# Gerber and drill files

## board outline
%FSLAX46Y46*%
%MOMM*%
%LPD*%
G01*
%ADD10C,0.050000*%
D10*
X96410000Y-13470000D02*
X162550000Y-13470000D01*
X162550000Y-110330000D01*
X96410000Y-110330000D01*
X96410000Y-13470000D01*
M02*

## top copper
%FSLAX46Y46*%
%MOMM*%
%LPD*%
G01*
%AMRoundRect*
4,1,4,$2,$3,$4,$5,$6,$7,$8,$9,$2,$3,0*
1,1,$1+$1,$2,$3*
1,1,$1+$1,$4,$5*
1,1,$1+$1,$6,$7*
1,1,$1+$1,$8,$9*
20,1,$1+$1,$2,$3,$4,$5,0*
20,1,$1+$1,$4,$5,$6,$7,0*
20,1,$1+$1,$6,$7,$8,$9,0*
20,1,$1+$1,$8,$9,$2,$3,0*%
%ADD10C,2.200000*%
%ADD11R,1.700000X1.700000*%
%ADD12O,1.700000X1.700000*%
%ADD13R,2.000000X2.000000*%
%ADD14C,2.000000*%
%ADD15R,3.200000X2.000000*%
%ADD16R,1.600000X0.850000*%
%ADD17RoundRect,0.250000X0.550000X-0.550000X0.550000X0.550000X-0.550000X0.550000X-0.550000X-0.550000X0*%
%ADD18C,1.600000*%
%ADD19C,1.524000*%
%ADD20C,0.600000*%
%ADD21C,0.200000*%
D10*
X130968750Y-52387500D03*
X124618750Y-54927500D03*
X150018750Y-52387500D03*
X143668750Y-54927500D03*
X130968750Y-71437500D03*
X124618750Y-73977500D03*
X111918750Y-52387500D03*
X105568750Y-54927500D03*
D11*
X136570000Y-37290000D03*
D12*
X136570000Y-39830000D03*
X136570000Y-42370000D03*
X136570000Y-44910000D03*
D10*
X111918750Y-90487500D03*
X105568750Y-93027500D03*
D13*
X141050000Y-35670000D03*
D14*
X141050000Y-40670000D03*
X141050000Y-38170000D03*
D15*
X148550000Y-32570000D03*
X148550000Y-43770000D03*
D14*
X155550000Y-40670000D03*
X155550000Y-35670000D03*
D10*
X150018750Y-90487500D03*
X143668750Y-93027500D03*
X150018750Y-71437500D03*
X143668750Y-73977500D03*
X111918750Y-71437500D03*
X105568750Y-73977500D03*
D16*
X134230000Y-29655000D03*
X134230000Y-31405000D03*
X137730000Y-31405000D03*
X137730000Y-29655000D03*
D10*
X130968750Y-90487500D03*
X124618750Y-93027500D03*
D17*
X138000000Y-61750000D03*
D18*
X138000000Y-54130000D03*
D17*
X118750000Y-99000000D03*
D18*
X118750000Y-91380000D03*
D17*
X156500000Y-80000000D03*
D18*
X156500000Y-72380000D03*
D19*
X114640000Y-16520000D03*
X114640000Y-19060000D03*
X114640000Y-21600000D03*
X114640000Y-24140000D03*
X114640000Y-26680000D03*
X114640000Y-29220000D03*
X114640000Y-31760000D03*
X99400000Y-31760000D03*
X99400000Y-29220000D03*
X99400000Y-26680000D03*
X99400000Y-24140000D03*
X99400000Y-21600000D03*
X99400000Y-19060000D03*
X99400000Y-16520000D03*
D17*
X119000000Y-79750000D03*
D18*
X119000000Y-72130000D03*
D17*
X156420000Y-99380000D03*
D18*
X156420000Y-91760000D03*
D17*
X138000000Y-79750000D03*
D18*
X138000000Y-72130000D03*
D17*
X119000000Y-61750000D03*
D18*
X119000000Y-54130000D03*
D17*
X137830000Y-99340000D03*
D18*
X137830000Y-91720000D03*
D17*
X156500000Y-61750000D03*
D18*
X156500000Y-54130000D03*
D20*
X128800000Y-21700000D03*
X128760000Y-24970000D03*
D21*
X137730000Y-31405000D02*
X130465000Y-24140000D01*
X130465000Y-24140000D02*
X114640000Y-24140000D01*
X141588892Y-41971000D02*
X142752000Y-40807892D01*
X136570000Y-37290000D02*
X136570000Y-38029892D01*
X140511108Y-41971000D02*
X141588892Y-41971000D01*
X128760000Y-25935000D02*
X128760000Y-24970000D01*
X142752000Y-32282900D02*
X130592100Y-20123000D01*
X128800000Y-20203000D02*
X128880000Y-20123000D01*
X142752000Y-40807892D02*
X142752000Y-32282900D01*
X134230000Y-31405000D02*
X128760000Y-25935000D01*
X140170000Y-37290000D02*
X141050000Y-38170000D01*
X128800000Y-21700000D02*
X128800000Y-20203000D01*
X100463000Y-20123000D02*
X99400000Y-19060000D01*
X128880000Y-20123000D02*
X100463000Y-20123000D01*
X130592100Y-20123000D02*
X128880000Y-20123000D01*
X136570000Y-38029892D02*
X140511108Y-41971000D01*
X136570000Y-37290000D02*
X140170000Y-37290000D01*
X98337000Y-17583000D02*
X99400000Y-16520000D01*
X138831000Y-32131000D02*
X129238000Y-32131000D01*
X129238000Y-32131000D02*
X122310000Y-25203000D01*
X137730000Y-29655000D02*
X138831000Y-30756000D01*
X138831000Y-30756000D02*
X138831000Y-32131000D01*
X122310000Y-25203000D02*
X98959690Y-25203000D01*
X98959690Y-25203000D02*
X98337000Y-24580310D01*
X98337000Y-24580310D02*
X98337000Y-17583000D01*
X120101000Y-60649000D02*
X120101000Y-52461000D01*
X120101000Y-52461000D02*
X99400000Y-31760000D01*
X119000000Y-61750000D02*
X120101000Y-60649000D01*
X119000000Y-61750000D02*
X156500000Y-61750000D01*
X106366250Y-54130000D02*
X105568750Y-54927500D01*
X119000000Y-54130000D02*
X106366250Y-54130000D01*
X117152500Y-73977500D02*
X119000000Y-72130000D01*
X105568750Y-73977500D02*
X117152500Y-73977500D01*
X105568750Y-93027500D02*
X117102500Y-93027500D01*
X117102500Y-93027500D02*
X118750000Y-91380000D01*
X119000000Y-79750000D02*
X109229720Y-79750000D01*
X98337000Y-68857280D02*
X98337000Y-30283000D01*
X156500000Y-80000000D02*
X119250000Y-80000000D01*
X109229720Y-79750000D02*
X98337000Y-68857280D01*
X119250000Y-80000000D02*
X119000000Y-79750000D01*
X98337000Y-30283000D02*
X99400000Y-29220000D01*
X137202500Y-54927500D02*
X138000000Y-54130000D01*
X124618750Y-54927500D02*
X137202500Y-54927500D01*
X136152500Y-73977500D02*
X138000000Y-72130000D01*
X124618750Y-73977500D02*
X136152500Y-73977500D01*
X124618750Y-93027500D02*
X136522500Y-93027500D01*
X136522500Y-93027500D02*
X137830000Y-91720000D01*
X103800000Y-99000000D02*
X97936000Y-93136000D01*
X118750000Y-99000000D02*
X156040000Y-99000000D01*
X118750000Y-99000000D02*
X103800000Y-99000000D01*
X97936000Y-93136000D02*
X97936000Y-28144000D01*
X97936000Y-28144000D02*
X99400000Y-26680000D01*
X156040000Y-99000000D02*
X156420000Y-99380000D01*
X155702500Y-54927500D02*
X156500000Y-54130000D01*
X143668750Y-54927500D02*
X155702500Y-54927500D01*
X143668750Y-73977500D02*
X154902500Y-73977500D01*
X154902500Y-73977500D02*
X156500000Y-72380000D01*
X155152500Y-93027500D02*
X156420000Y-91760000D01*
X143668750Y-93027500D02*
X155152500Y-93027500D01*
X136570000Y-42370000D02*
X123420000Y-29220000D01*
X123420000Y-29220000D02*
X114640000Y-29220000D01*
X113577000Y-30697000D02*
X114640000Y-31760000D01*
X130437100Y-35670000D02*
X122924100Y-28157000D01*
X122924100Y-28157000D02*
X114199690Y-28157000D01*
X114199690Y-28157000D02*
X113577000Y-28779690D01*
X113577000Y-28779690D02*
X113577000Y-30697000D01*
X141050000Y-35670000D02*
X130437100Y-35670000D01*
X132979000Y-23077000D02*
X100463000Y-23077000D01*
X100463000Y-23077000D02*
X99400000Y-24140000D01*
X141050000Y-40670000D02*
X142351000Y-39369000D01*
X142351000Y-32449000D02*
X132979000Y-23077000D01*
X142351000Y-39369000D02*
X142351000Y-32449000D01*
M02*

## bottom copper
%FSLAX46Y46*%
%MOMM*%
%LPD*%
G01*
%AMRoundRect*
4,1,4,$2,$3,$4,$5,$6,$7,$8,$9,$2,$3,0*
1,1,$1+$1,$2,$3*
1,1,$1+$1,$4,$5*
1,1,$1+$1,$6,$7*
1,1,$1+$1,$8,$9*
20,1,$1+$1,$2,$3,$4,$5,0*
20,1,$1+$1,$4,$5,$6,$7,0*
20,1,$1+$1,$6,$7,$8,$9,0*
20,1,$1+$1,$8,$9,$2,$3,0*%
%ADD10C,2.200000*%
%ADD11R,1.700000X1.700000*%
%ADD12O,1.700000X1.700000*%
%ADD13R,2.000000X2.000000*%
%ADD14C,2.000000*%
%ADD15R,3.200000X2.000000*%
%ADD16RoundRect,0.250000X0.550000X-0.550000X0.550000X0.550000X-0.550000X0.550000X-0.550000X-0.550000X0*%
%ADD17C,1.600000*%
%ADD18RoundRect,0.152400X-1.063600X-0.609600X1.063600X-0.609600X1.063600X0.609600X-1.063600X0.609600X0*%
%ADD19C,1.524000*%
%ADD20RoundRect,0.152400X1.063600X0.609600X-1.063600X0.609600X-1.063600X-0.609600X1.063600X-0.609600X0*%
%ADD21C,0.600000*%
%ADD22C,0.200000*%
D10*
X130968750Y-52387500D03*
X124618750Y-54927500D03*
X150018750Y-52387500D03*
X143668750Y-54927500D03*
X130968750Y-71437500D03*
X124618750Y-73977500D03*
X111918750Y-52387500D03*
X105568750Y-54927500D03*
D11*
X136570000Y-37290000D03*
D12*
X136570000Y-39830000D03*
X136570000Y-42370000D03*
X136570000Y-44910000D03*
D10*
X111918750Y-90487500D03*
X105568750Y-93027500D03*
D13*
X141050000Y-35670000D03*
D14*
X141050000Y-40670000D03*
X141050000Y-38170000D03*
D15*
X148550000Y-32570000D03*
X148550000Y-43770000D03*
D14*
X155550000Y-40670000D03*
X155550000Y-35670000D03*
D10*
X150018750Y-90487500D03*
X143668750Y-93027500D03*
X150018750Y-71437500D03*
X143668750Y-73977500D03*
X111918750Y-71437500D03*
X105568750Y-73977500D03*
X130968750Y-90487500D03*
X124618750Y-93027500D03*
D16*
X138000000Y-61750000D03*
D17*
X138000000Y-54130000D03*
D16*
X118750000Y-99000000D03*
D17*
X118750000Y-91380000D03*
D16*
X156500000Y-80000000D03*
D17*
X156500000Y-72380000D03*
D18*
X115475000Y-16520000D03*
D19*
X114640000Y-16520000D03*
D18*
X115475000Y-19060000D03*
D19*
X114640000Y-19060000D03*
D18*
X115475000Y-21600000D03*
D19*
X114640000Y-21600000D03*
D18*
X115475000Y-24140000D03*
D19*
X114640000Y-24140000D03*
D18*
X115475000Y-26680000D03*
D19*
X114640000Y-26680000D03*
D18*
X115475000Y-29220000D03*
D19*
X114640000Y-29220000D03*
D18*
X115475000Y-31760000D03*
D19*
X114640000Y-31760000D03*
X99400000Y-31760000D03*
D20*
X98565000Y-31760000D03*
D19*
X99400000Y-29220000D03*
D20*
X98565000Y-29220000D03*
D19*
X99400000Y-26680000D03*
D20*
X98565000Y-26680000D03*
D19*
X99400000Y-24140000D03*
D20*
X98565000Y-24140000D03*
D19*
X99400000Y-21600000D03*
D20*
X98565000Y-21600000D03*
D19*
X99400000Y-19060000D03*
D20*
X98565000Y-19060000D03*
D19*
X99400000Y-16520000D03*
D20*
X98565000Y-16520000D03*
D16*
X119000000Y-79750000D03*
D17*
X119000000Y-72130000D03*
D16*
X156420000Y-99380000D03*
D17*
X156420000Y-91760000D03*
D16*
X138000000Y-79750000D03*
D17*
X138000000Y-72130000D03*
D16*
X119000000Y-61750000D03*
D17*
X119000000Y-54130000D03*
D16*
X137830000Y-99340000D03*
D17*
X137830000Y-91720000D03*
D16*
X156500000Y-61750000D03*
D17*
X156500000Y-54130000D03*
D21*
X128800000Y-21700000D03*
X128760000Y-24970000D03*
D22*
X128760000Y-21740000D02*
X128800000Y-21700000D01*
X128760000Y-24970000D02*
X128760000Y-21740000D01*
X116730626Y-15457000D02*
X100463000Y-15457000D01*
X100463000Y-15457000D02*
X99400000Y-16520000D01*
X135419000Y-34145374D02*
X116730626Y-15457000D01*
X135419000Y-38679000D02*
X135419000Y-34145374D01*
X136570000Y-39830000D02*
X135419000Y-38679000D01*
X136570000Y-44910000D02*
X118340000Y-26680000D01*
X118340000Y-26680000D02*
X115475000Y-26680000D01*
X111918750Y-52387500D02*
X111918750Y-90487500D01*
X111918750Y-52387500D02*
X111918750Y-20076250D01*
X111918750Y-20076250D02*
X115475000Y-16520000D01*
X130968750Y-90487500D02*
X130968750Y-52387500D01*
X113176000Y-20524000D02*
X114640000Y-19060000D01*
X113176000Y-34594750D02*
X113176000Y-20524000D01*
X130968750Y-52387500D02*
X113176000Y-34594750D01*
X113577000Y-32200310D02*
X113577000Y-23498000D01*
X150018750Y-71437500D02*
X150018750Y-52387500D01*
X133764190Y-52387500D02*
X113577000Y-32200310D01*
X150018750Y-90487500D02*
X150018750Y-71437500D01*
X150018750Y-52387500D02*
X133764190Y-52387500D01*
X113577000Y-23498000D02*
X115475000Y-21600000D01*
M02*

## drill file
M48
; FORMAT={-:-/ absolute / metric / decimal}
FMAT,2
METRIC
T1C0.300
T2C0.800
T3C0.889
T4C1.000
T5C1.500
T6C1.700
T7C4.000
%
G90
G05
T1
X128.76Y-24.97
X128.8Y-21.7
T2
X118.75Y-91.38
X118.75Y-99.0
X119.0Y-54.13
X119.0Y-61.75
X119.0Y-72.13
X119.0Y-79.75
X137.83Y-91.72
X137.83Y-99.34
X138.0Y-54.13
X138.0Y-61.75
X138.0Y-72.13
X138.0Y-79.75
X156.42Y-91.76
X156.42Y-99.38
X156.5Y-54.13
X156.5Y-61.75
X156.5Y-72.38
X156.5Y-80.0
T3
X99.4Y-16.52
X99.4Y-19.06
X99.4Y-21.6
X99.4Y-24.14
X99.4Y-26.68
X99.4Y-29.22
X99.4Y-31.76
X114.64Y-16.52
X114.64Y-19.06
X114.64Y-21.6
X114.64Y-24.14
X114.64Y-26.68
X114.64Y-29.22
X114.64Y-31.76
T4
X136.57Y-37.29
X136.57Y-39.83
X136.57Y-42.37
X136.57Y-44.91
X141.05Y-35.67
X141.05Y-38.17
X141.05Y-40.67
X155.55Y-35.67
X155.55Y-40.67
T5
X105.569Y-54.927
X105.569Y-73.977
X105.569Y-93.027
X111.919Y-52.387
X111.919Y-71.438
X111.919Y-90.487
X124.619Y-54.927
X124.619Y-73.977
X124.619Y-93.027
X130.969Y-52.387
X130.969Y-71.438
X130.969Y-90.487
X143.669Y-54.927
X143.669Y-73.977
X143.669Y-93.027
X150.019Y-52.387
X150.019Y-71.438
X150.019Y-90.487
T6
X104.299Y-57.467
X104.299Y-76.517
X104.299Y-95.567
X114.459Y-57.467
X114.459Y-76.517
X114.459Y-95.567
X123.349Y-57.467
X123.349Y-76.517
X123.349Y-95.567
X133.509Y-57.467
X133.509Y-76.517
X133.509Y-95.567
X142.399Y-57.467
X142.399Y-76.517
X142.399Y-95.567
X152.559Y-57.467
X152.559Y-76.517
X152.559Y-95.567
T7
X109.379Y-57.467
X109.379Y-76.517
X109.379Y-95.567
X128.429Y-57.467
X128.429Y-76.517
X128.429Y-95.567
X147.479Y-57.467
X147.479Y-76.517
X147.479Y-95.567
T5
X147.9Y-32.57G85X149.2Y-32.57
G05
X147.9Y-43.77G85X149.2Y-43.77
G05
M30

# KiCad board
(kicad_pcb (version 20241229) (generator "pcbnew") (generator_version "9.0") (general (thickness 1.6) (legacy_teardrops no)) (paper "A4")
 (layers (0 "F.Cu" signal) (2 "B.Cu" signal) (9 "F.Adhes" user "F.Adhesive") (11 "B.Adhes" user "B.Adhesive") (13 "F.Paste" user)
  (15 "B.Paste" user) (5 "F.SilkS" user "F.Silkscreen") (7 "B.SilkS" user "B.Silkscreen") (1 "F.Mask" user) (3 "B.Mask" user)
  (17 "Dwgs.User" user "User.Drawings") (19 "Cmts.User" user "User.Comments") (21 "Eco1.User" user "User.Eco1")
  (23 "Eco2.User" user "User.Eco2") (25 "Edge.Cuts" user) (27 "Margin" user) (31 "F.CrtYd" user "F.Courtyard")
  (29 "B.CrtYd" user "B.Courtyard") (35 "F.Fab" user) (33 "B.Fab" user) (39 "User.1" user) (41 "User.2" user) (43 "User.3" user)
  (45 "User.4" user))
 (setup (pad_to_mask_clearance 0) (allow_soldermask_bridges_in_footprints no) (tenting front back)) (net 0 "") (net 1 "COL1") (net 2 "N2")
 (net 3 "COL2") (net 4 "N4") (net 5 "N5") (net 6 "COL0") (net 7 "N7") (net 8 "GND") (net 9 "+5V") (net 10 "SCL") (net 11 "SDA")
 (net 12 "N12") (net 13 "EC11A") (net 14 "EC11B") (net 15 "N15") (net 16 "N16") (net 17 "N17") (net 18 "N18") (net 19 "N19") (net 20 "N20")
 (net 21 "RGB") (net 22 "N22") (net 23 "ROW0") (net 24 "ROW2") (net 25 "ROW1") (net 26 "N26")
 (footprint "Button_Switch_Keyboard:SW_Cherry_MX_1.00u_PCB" (layer "F.Cu") (at 130.96875 52.3875)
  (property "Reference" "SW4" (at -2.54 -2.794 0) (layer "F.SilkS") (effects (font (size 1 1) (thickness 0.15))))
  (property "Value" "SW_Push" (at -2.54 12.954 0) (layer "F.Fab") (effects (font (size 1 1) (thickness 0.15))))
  (pad "" np_thru_hole circle (at -7.62 5.08) (size 1.7 1.7) (drill 1.7) (layers "*.Cu" "*.Mask"))
  (pad "" np_thru_hole circle (at -2.54 5.08) (size 4 4) (drill 4) (layers "*.Cu" "*.Mask"))
  (pad "" np_thru_hole circle (at 2.54 5.08) (size 1.7 1.7) (drill 1.7) (layers "*.Cu" "*.Mask"))
  (pad "1" thru_hole circle (at 0 0) (size 2.2 2.2) (drill 1.5) (layers "*.Cu" "*.Mask") (remove_unused_layers no) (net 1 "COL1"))
  (pad "2" thru_hole circle (at -6.35 2.54) (size 2.2 2.2) (drill 1.5) (layers "*.Cu" "*.Mask") (remove_unused_layers no) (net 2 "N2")))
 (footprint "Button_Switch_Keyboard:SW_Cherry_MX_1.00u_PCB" (layer "F.Cu") (at 150.01875 52.3875)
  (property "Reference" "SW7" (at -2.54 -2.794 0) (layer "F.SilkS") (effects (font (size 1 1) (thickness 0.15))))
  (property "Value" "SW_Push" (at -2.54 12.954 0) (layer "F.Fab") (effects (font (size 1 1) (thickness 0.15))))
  (pad "" np_thru_hole circle (at -7.62 5.08) (size 1.7 1.7) (drill 1.7) (layers "*.Cu" "*.Mask"))
  (pad "" np_thru_hole circle (at -2.54 5.08) (size 4 4) (drill 4) (layers "*.Cu" "*.Mask"))
  (pad "" np_thru_hole circle (at 2.54 5.08) (size 1.7 1.7) (drill 1.7) (layers "*.Cu" "*.Mask"))
  (pad "1" thru_hole circle (at 0 0) (size 2.2 2.2) (drill 1.5) (layers "*.Cu" "*.Mask") (remove_unused_layers no) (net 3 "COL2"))
  (pad "2" thru_hole circle (at -6.35 2.54) (size 2.2 2.2) (drill 1.5) (layers "*.Cu" "*.Mask") (remove_unused_layers no) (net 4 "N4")))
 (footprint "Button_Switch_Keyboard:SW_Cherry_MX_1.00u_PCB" (layer "F.Cu") (at 130.96875 71.4375)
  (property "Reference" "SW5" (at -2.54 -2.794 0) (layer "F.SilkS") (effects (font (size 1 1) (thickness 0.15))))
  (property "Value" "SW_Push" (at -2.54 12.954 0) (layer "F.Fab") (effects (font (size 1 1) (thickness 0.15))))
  (pad "" np_thru_hole circle (at -7.62 5.08) (size 1.7 1.7) (drill 1.7) (layers "*.Cu" "*.Mask"))
  (pad "" np_thru_hole circle (at -2.54 5.08) (size 4 4) (drill 4) (layers "*.Cu" "*.Mask"))
  (pad "" np_thru_hole circle (at 2.54 5.08) (size 1.7 1.7) (drill 1.7) (layers "*.Cu" "*.Mask"))
  (pad "1" thru_hole circle (at 0 0) (size 2.2 2.2) (drill 1.5) (layers "*.Cu" "*.Mask") (remove_unused_layers no) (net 1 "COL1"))
  (pad "2" thru_hole circle (at -6.35 2.54) (size 2.2 2.2) (drill 1.5) (layers "*.Cu" "*.Mask") (remove_unused_layers no) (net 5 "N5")))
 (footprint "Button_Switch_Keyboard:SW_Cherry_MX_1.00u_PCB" (layer "F.Cu") (at 111.91875 52.3875)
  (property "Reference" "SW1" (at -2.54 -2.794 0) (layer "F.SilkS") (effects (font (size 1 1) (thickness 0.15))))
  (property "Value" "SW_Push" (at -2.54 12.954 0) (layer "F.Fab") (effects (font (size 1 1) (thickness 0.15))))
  (pad "" np_thru_hole circle (at -7.62 5.08) (size 1.7 1.7) (drill 1.7) (layers "*.Cu" "*.Mask"))
  (pad "" np_thru_hole circle (at -2.54 5.08) (size 4 4) (drill 4) (layers "*.Cu" "*.Mask"))
  (pad "" np_thru_hole circle (at 2.54 5.08) (size 1.7 1.7) (drill 1.7) (layers "*.Cu" "*.Mask"))
  (pad "1" thru_hole circle (at 0 0) (size 2.2 2.2) (drill 1.5) (layers "*.Cu" "*.Mask") (remove_unused_layers no) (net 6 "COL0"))
  (pad "2" thru_hole circle (at -6.35 2.54) (size 2.2 2.2) (drill 1.5) (layers "*.Cu" "*.Mask") (remove_unused_layers no) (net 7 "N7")))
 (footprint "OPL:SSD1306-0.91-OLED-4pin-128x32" (layer "F.Cu") (at 100.07 35.1)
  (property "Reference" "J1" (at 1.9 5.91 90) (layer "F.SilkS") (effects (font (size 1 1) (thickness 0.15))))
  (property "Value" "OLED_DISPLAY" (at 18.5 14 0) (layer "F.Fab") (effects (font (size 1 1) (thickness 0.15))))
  (pad "1" thru_hole rect (at 36.5 2.19) (size 1.7 1.7) (drill 1) (layers "*.Cu" "*.Mask") (remove_unused_layers no) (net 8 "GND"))
  (pad "2" thru_hole oval (at 36.5 4.73) (size 1.7 1.7) (drill 1) (layers "*.Cu" "*.Mask") (remove_unused_layers no) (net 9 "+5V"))
  (pad "3" thru_hole oval (at 36.5 7.27) (size 1.7 1.7) (drill 1) (layers "*.Cu" "*.Mask") (remove_unused_layers no) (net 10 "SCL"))
  (pad "4" thru_hole oval (at 36.5 9.81) (size 1.7 1.7) (drill 1) (layers "*.Cu" "*.Mask") (remove_unused_layers no) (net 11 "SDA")))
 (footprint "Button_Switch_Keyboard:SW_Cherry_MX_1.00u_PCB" (layer "F.Cu") (at 111.91875 90.4875)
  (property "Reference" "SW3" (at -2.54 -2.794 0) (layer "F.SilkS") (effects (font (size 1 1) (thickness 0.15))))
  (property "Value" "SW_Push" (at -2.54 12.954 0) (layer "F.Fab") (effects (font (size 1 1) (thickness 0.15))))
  (pad "" np_thru_hole circle (at -7.62 5.08) (size 1.7 1.7) (drill 1.7) (layers "*.Cu" "*.Mask"))
  (pad "" np_thru_hole circle (at -2.54 5.08) (size 4 4) (drill 4) (layers "*.Cu" "*.Mask"))
  (pad "" np_thru_hole circle (at 2.54 5.08) (size 1.7 1.7) (drill 1.7) (layers "*.Cu" "*.Mask"))
  (pad "1" thru_hole circle (at 0 0) (size 2.2 2.2) (drill 1.5) (layers "*.Cu" "*.Mask") (remove_unused_layers no) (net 6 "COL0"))
  (pad "2" thru_hole circle (at -6.35 2.54) (size 2.2 2.2) (drill 1.5) (layers "*.Cu" "*.Mask") (remove_unused_layers no) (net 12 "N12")))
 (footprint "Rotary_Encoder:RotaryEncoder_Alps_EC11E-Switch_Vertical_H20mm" (layer "F.Cu") (at 141.05 35.67)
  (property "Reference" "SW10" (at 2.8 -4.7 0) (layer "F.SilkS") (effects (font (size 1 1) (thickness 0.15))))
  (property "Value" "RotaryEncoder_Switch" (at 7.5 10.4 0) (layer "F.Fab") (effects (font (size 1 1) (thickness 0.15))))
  (pad "A" thru_hole rect (at 0 0) (size 2 2) (drill 1) (layers "*.Cu" "*.Mask") (remove_unused_layers no) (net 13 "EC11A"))
  (pad "B" thru_hole circle (at 0 5) (size 2 2) (drill 1) (layers "*.Cu" "*.Mask") (remove_unused_layers no) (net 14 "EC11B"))
  (pad "C" thru_hole circle (at 0 2.5) (size 2 2) (drill 1) (layers "*.Cu" "*.Mask") (remove_unused_layers no) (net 8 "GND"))
  (pad "MP" thru_hole rect (at 7.5 -3.1) (size 3.2 2) (drill oval 2.8 1.5) (layers "*.Cu" "*.Mask") (remove_unused_layers no))
  (pad "MP" thru_hole rect (at 7.5 8.1) (size 3.2 2) (drill oval 2.8 1.5) (layers "*.Cu" "*.Mask") (remove_unused_layers no))
  (pad "S1" thru_hole circle (at 14.5 5) (size 2 2) (drill 1) (layers "*.Cu" "*.Mask") (remove_unused_layers no) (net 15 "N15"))
  (pad "S2" thru_hole circle (at 14.5 0) (size 2 2) (drill 1) (layers "*.Cu" "*.Mask") (remove_unused_layers no) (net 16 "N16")))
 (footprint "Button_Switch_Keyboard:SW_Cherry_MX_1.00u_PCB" (layer "F.Cu") (at 150.01875 90.4875)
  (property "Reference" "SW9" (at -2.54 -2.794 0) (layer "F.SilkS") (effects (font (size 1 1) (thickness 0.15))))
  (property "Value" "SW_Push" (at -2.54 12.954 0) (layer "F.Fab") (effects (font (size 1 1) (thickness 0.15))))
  (pad "" np_thru_hole circle (at -7.62 5.08) (size 1.7 1.7) (drill 1.7) (layers "*.Cu" "*.Mask"))
  (pad "" np_thru_hole circle (at -2.54 5.08) (size 4 4) (drill 4) (layers "*.Cu" "*.Mask"))
  (pad "" np_thru_hole circle (at 2.54 5.08) (size 1.7 1.7) (drill 1.7) (layers "*.Cu" "*.Mask"))
  (pad "1" thru_hole circle (at 0 0) (size 2.2 2.2) (drill 1.5) (layers "*.Cu" "*.Mask") (remove_unused_layers no) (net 3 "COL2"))
  (pad "2" thru_hole circle (at -6.35 2.54) (size 2.2 2.2) (drill 1.5) (layers "*.Cu" "*.Mask") (remove_unused_layers no) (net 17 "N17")))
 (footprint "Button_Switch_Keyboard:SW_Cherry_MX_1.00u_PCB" (layer "F.Cu") (at 150.01875 71.4375)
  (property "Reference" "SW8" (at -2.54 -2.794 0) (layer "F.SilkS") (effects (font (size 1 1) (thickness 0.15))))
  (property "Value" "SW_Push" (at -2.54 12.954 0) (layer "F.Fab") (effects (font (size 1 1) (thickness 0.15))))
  (pad "" np_thru_hole circle (at -7.62 5.08) (size 1.7 1.7) (drill 1.7) (layers "*.Cu" "*.Mask"))
  (pad "" np_thru_hole circle (at -2.54 5.08) (size 4 4) (drill 4) (layers "*.Cu" "*.Mask"))
  (pad "" np_thru_hole circle (at 2.54 5.08) (size 1.7 1.7) (drill 1.7) (layers "*.Cu" "*.Mask"))
  (pad "1" thru_hole circle (at 0 0) (size 2.2 2.2) (drill 1.5) (layers "*.Cu" "*.Mask") (remove_unused_layers no) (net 3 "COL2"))
  (pad "2" thru_hole circle (at -6.35 2.54) (size 2.2 2.2) (drill 1.5) (layers "*.Cu" "*.Mask") (remove_unused_layers no) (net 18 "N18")))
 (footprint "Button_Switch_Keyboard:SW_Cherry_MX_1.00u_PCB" (layer "F.Cu") (at 111.91875 71.4375)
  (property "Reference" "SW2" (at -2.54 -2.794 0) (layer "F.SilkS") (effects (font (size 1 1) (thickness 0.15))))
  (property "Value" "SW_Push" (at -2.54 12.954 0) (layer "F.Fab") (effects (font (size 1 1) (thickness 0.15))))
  (pad "" np_thru_hole circle (at -7.62 5.08) (size 1.7 1.7) (drill 1.7) (layers "*.Cu" "*.Mask"))
  (pad "" np_thru_hole circle (at -2.54 5.08) (size 4 4) (drill 4) (layers "*.Cu" "*.Mask"))
  (pad "" np_thru_hole circle (at 2.54 5.08) (size 1.7 1.7) (drill 1.7) (layers "*.Cu" "*.Mask"))
  (pad "1" thru_hole circle (at 0 0) (size 2.2 2.2) (drill 1.5) (layers "*.Cu" "*.Mask") (remove_unused_layers no) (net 6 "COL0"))
  (pad "2" thru_hole circle (at -6.35 2.54) (size 2.2 2.2) (drill 1.5) (layers "*.Cu" "*.Mask") (remove_unused_layers no) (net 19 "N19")))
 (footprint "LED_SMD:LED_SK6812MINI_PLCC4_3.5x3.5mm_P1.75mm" (layer "F.Cu") (at 135.98 30.53)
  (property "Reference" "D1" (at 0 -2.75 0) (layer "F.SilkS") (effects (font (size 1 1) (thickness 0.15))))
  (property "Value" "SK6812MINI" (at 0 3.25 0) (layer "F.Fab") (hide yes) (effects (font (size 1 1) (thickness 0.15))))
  (pad "1" smd rect (at -1.75 -0.875) (size 1.6 0.85) (layers "F.Cu" "F.Mask" "F.Paste") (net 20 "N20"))
  (pad "2" smd rect (at -1.75 0.875) (size 1.6 0.85) (layers "F.Cu" "F.Mask" "F.Paste") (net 8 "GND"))
  (pad "3" smd rect (at 1.75 0.875) (size 1.6 0.85) (layers "F.Cu" "F.Mask" "F.Paste") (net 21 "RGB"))
  (pad "4" smd rect (at 1.75 -0.875) (size 1.6 0.85) (layers "F.Cu" "F.Mask" "F.Paste") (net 9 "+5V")))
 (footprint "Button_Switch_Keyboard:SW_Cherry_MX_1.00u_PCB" (layer "F.Cu") (at 130.96875 90.4875)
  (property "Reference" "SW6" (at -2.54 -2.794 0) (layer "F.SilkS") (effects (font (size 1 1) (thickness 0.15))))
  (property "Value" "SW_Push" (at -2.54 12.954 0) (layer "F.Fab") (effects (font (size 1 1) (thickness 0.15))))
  (pad "" np_thru_hole circle (at -7.62 5.08) (size 1.7 1.7) (drill 1.7) (layers "*.Cu" "*.Mask"))
  (pad "" np_thru_hole circle (at -2.54 5.08) (size 4 4) (drill 4) (layers "*.Cu" "*.Mask"))
  (pad "" np_thru_hole circle (at 2.54 5.08) (size 1.7 1.7) (drill 1.7) (layers "*.Cu" "*.Mask"))
  (pad "1" thru_hole circle (at 0 0) (size 2.2 2.2) (drill 1.5) (layers "*.Cu" "*.Mask") (remove_unused_layers no) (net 1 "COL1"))
  (pad "2" thru_hole circle (at -6.35 2.54) (size 2.2 2.2) (drill 1.5) (layers "*.Cu" "*.Mask") (remove_unused_layers no) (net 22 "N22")))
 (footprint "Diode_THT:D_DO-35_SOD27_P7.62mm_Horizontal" (layer "B.Cu") (at 138 61.75 90)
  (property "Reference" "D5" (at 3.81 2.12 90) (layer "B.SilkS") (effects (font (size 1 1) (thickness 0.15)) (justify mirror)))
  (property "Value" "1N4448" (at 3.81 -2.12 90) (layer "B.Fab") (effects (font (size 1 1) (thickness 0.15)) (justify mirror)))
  (pad "1" thru_hole roundrect (at 0 0 90) (size 1.6 1.6) (drill 0.8) (layers "*.Cu" "*.Mask") (remove_unused_layers no)
   (roundrect_rratio 0.15625) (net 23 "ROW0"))
  (pad "2" thru_hole circle (at 7.62 0 90) (size 1.6 1.6) (drill 0.8) (layers "*.Cu" "*.Mask") (remove_unused_layers no) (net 2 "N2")))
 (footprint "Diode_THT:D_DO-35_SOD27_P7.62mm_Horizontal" (layer "B.Cu") (at 118.75 99 90)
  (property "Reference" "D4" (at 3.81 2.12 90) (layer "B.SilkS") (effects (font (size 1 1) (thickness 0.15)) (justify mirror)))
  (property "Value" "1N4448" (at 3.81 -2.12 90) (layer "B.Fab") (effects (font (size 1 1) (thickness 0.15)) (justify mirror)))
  (pad "1" thru_hole roundrect (at 0 0 90) (size 1.6 1.6) (drill 0.8) (layers "*.Cu" "*.Mask") (remove_unused_layers no)
   (roundrect_rratio 0.15625) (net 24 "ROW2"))
  (pad "2" thru_hole circle (at 7.62 0 90) (size 1.6 1.6) (drill 0.8) (layers "*.Cu" "*.Mask") (remove_unused_layers no) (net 12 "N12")))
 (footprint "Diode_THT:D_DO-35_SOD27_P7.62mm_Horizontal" (layer "B.Cu") (at 156.5 80 90)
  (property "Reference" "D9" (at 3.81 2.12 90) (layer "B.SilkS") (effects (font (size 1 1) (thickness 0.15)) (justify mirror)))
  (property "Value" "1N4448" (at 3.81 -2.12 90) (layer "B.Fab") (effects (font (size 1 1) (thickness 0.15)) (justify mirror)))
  (pad "1" thru_hole roundrect (at 0 0 90) (size 1.6 1.6) (drill 0.8) (layers "*.Cu" "*.Mask") (remove_unused_layers no)
   (roundrect_rratio 0.15625) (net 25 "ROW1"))
  (pad "2" thru_hole circle (at 7.62 0 90) (size 1.6 1.6) (drill 0.8) (layers "*.Cu" "*.Mask") (remove_unused_layers no) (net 18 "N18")))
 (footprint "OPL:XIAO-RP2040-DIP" (layer "B.Cu") (at 107.02 24.14 180)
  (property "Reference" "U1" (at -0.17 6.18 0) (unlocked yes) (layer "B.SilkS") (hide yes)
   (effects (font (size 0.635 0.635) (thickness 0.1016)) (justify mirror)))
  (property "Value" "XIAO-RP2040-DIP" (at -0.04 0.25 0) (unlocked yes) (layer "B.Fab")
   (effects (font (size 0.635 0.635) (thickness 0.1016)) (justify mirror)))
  (pad "1" smd roundrect (at -8.455 7.62) (size 2.432 1.524) (layers "B.Cu" "B.Mask") (roundrect_rratio 0.1) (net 6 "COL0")
   (thermal_bridge_angle 45))
  (pad "1" thru_hole circle (at -7.62 7.62) (size 1.524 1.524) (drill 0.889) (layers "*.Cu" "*.Mask") (remove_unused_layers no)
   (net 6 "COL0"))
  (pad "2" smd roundrect (at -8.455 5.08) (size 2.432 1.524) (layers "B.Cu" "B.Mask") (roundrect_rratio 0.1) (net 1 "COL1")
   (thermal_bridge_angle 45))
  (pad "2" thru_hole circle (at -7.62 5.08) (size 1.524 1.524) (drill 0.889) (layers "*.Cu" "*.Mask") (remove_unused_layers no)
   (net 1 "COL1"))
  (pad "3" smd roundrect (at -8.455 2.54) (size 2.432 1.524) (layers "B.Cu" "B.Mask") (roundrect_rratio 0.1) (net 3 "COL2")
   (thermal_bridge_angle 45))
  (pad "3" thru_hole circle (at -7.62 2.54) (size 1.524 1.524) (drill 0.889) (layers "*.Cu" "*.Mask") (remove_unused_layers no)
   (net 3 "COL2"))
  (pad "4" smd roundrect (at -8.455 0) (size 2.432 1.524) (layers "B.Cu" "B.Mask") (roundrect_rratio 0.1) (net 21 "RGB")
   (thermal_bridge_angle 45))
  (pad "4" thru_hole circle (at -7.62 0) (size 1.524 1.524) (drill 0.889) (layers "*.Cu" "*.Mask") (remove_unused_layers no) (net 21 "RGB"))
  (pad "5" smd roundrect (at -8.455 -2.54) (size 2.432 1.524) (layers "B.Cu" "B.Mask") (roundrect_rratio 0.1) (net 11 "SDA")
   (thermal_bridge_angle 45))
  (pad "5" thru_hole circle (at -7.62 -2.54) (size 1.524 1.524) (drill 0.889) (layers "*.Cu" "*.Mask") (remove_unused_layers no)
   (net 11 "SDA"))
  (pad "6" smd roundrect (at -8.455 -5.08) (size 2.432 1.524) (layers "B.Cu" "B.Mask") (roundrect_rratio 0.1) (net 10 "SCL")
   (thermal_bridge_angle 45))
  (pad "6" thru_hole circle (at -7.62 -5.08) (size 1.524 1.524) (drill 0.889) (layers "*.Cu" "*.Mask") (remove_unused_layers no)
   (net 10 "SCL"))
  (pad "7" smd roundrect (at -8.455 -7.62) (size 2.432 1.524) (layers "B.Cu" "B.Mask") (roundrect_rratio 0.1) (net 13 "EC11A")
   (thermal_bridge_angle 45))
  (pad "7" thru_hole circle (at -7.62 -7.62) (size 1.524 1.524) (drill 0.889) (layers "*.Cu" "*.Mask") (remove_unused_layers no)
   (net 13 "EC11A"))
  (pad "8" thru_hole circle (at 7.62 -7.62 180) (size 1.524 1.524) (drill 0.889) (layers "*.Cu" "*.Mask") (remove_unused_layers no)
   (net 23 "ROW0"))
  (pad "8" smd roundrect (at 8.455 -7.62 180) (size 2.432 1.524) (layers "B.Cu" "B.Mask") (roundrect_rratio 0.1) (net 23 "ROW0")
   (thermal_bridge_angle 45))
  (pad "9" thru_hole circle (at 7.62 -5.08 180) (size 1.524 1.524) (drill 0.889) (layers "*.Cu" "*.Mask") (remove_unused_layers no)
   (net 25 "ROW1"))
  (pad "9" smd roundrect (at 8.455 -5.08 180) (size 2.432 1.524) (layers "B.Cu" "B.Mask") (roundrect_rratio 0.1) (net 25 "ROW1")
   (thermal_bridge_angle 45))
  (pad "10" thru_hole circle (at 7.62 -2.54 180) (size 1.524 1.524) (drill 0.889) (layers "*.Cu" "*.Mask") (remove_unused_layers no)
   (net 24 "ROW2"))
  (pad "10" smd roundrect (at 8.455 -2.54 180) (size 2.432 1.524) (layers "B.Cu" "B.Mask") (roundrect_rratio 0.1) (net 24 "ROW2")
   (thermal_bridge_angle 45))
  (pad "11" thru_hole circle (at 7.62 0 180) (size 1.524 1.524) (drill 0.889) (layers "*.Cu" "*.Mask") (remove_unused_layers no)
   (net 14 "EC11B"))
  (pad "11" smd roundrect (at 8.455 0 180) (size 2.432 1.524) (layers "B.Cu" "B.Mask") (roundrect_rratio 0.1) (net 14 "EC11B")
   (thermal_bridge_angle 45))
  (pad "12" thru_hole circle (at 7.62 2.54 180) (size 1.524 1.524) (drill 0.889) (layers "*.Cu" "*.Mask") (remove_unused_layers no)
   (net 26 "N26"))
  (pad "12" smd roundrect (at 8.455 2.54 180) (size 2.432 1.524) (layers "B.Cu" "B.Mask") (roundrect_rratio 0.1) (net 26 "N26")
   (thermal_bridge_angle 45))
  (pad "13" thru_hole circle (at 7.62 5.08 180) (size 1.524 1.524) (drill 0.889) (layers "*.Cu" "*.Mask") (remove_unused_layers no)
   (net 8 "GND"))
  (pad "13" smd roundrect (at 8.455 5.08 180) (size 2.432 1.524) (layers "B.Cu" "B.Mask") (roundrect_rratio 0.1) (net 8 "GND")
   (thermal_bridge_angle 45))
  (pad "14" thru_hole circle (at 7.62 7.62 180) (size 1.524 1.524) (drill 0.889) (layers "*.Cu" "*.Mask") (remove_unused_layers no)
   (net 9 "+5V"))
  (pad "14" smd roundrect (at 8.455 7.62 180) (size 2.432 1.524) (layers "B.Cu" "B.Mask") (roundrect_rratio 0.1) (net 9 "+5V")
   (thermal_bridge_angle 45)))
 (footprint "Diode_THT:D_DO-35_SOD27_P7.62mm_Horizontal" (layer "B.Cu") (at 119 79.75 90)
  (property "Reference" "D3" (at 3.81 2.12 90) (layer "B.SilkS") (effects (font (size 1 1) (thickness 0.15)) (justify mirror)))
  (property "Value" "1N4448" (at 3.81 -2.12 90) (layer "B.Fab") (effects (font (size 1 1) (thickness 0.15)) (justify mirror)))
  (pad "1" thru_hole roundrect (at 0 0 90) (size 1.6 1.6) (drill 0.8) (layers "*.Cu" "*.Mask") (remove_unused_layers no)
   (roundrect_rratio 0.15625) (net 25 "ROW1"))
  (pad "2" thru_hole circle (at 7.62 0 90) (size 1.6 1.6) (drill 0.8) (layers "*.Cu" "*.Mask") (remove_unused_layers no) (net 19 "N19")))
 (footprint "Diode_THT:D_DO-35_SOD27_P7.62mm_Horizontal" (layer "B.Cu") (at 156.42 99.38 90)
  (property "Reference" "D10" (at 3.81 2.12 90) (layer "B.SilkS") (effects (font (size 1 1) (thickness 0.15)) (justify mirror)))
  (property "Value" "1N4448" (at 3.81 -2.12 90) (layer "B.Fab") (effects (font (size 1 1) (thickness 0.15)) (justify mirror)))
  (pad "1" thru_hole roundrect (at 0 0 90) (size 1.6 1.6) (drill 0.8) (layers "*.Cu" "*.Mask") (remove_unused_layers no)
   (roundrect_rratio 0.15625) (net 24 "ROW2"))
  (pad "2" thru_hole circle (at 7.62 0 90) (size 1.6 1.6) (drill 0.8) (layers "*.Cu" "*.Mask") (remove_unused_layers no) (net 17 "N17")))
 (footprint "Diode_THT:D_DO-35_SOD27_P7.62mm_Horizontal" (layer "B.Cu") (at 138 79.75 90)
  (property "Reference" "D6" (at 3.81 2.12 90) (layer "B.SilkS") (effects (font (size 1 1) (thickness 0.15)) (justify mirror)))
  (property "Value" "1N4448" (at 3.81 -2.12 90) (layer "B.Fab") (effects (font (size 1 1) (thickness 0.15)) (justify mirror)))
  (pad "1" thru_hole roundrect (at 0 0 90) (size 1.6 1.6) (drill 0.8) (layers "*.Cu" "*.Mask") (remove_unused_layers no)
   (roundrect_rratio 0.15625) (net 25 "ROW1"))
  (pad "2" thru_hole circle (at 7.62 0 90) (size 1.6 1.6) (drill 0.8) (layers "*.Cu" "*.Mask") (remove_unused_layers no) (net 5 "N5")))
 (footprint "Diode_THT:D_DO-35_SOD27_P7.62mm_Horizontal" (layer "B.Cu") (at 119 61.75 90)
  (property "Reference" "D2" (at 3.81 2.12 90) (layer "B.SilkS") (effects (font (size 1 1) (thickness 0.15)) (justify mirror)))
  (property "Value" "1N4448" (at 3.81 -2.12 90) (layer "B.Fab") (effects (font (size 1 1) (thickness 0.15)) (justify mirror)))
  (pad "1" thru_hole roundrect (at 0 0 90) (size 1.6 1.6) (drill 0.8) (layers "*.Cu" "*.Mask") (remove_unused_layers no)
   (roundrect_rratio 0.15625) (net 23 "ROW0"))
  (pad "2" thru_hole circle (at 7.62 0 90) (size 1.6 1.6) (drill 0.8) (layers "*.Cu" "*.Mask") (remove_unused_layers no) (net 7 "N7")))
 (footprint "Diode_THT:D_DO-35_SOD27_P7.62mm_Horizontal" (layer "B.Cu") (at 137.83 99.34 90)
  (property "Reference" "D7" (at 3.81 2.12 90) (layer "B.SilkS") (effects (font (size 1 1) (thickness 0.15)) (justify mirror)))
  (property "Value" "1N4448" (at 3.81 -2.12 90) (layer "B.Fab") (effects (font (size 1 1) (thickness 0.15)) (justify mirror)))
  (pad "1" thru_hole roundrect (at 0 0 90) (size 1.6 1.6) (drill 0.8) (layers "*.Cu" "*.Mask") (remove_unused_layers no)
   (roundrect_rratio 0.15625) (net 24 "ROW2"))
  (pad "2" thru_hole circle (at 7.62 0 90) (size 1.6 1.6) (drill 0.8) (layers "*.Cu" "*.Mask") (remove_unused_layers no) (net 22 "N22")))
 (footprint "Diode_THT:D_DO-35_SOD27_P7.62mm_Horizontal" (layer "B.Cu") (at 156.5 61.75 90)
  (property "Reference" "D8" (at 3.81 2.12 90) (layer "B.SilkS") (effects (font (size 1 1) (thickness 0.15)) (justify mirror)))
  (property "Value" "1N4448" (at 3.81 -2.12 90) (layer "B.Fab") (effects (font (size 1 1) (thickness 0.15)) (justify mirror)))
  (pad "1" thru_hole roundrect (at 0 0 90) (size 1.6 1.6) (drill 0.8) (layers "*.Cu" "*.Mask") (remove_unused_layers no)
   (roundrect_rratio 0.15625) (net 23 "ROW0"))
  (pad "2" thru_hole circle (at 7.62 0 90) (size 1.6 1.6) (drill 0.8) (layers "*.Cu" "*.Mask") (remove_unused_layers no) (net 4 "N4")))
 (gr_rect (start 96.41 13.47) (end 162.55 110.33) (stroke (width 0.05) (type default)) (fill no) (layer "Edge.Cuts"))
 (segment (start 137.73 31.405) (end 130.465 24.14) (width 0.2) (layer "F.Cu") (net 21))
 (segment (start 130.465 24.14) (end 114.64 24.14) (width 0.2) (layer "F.Cu") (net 21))
 (segment (start 141.588892 41.971) (end 142.752 40.807892) (width 0.2) (layer "F.Cu") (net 8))
 (segment (start 136.57 37.29) (end 136.57 38.029892) (width 0.2) (layer "F.Cu") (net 8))
 (segment (start 140.511108 41.971) (end 141.588892 41.971) (width 0.2) (layer "F.Cu") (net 8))
 (segment (start 128.76 25.935) (end 128.76 24.97) (width 0.2) (layer "F.Cu") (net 8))
 (segment (start 142.752 32.2829) (end 130.5921 20.123) (width 0.2) (layer "F.Cu") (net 8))
 (segment (start 128.8 20.203) (end 128.88 20.123) (width 0.2) (layer "F.Cu") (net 8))
 (segment (start 142.752 40.807892) (end 142.752 32.2829) (width 0.2) (layer "F.Cu") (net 8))
 (segment (start 134.23 31.405) (end 128.76 25.935) (width 0.2) (layer "F.Cu") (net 8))
 (segment (start 140.17 37.29) (end 141.05 38.17) (width 0.2) (layer "F.Cu") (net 8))
 (segment (start 128.8 21.7) (end 128.8 20.203) (width 0.2) (layer "F.Cu") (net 8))
 (segment (start 100.463 20.123) (end 99.4 19.06) (width 0.2) (layer "F.Cu") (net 8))
 (segment (start 128.88 20.123) (end 100.463 20.123) (width 0.2) (layer "F.Cu") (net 8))
 (segment (start 130.5921 20.123) (end 128.88 20.123) (width 0.2) (layer "F.Cu") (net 8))
 (segment (start 136.57 38.029892) (end 140.511108 41.971) (width 0.2) (layer "F.Cu") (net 8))
 (segment (start 136.57 37.29) (end 140.17 37.29) (width 0.2) (layer "F.Cu") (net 8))
 (via (at 128.8 21.7) (size 0.6) (drill 0.3) (layers "F.Cu" "B.Cu") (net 8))
 (via (at 128.76 24.97) (size 0.6) (drill 0.3) (layers "F.Cu" "B.Cu") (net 8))
 (segment (start 128.76 21.74) (end 128.8 21.7) (width 0.2) (layer "B.Cu") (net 8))
 (segment (start 128.76 24.97) (end 128.76 21.74) (width 0.2) (layer "B.Cu") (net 8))
 (segment (start 98.337 17.583) (end 99.4 16.52) (width 0.2) (layer "F.Cu") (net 9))
 (segment (start 138.831 32.131) (end 129.238 32.131) (width 0.2) (layer "F.Cu") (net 9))
 (segment (start 129.238 32.131) (end 122.31 25.203) (width 0.2) (layer "F.Cu") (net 9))
 (segment (start 137.73 29.655) (end 138.831 30.756) (width 0.2) (layer "F.Cu") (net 9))
 (segment (start 138.831 30.756) (end 138.831 32.131) (width 0.2) (layer "F.Cu") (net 9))
 (segment (start 122.31 25.203) (end 98.95969 25.203) (width 0.2) (layer "F.Cu") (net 9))
 (segment (start 98.95969 25.203) (end 98.337 24.58031) (width 0.2) (layer "F.Cu") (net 9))
 (segment (start 98.337 24.58031) (end 98.337 17.583) (width 0.2) (layer "F.Cu") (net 9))
 (segment (start 116.730626 15.457) (end 100.463 15.457) (width 0.2) (layer "B.Cu") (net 9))
 (segment (start 100.463 15.457) (end 99.4 16.52) (width 0.2) (layer "B.Cu") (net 9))
 (segment (start 135.419 34.145374) (end 116.730626 15.457) (width 0.2) (layer "B.Cu") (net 9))
 (segment (start 135.419 38.679) (end 135.419 34.145374) (width 0.2) (layer "B.Cu") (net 9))
 (segment (start 136.57 39.83) (end 135.419 38.679) (width 0.2) (layer "B.Cu") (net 9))
 (segment (start 120.101 60.649) (end 120.101 52.461) (width 0.2) (layer "F.Cu") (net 23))
 (segment (start 120.101 52.461) (end 99.4 31.76) (width 0.2) (layer "F.Cu") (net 23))
 (segment (start 119 61.75) (end 120.101 60.649) (width 0.2) (layer "F.Cu") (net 23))
 (segment (start 119 61.75) (end 156.5 61.75) (width 0.2) (layer "F.Cu") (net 23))
 (segment (start 106.36625 54.13) (end 105.56875 54.9275) (width 0.2) (layer "F.Cu") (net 7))
 (segment (start 119 54.13) (end 106.36625 54.13) (width 0.2) (layer "F.Cu") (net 7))
 (segment (start 117.1525 73.9775) (end 119 72.13) (width 0.2) (layer "F.Cu") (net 19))
 (segment (start 105.56875 73.9775) (end 117.1525 73.9775) (width 0.2) (layer "F.Cu") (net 19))
 (segment (start 105.56875 93.0275) (end 117.1025 93.0275) (width 0.2) (layer "F.Cu") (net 12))
 (segment (start 117.1025 93.0275) (end 118.75 91.38) (width 0.2) (layer "F.Cu") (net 12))
 (segment (start 119 79.75) (end 109.22972 79.75) (width 0.2) (layer "F.Cu") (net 25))
 (segment (start 98.337 68.85728) (end 98.337 30.283) (width 0.2) (layer "F.Cu") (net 25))
 (segment (start 156.5 80) (end 119.25 80) (width 0.2) (layer "F.Cu") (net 25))
 (segment (start 109.22972 79.75) (end 98.337 68.85728) (width 0.2) (layer "F.Cu") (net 25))
 (segment (start 119.25 80) (end 119 79.75) (width 0.2) (layer "F.Cu") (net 25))
 (segment (start 98.337 30.283) (end 99.4 29.22) (width 0.2) (layer "F.Cu") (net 25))
 (segment (start 137.2025 54.9275) (end 138 54.13) (width 0.2) (layer "F.Cu") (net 2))
 (segment (start 124.61875 54.9275) (end 137.2025 54.9275) (width 0.2) (layer "F.Cu") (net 2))
 (segment (start 136.1525 73.9775) (end 138 72.13) (width 0.2) (layer "F.Cu") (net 5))
 (segment (start 124.61875 73.9775) (end 136.1525 73.9775) (width 0.2) (layer "F.Cu") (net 5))
 (segment (start 124.61875 93.0275) (end 136.5225 93.0275) (width 0.2) (layer "F.Cu") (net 22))
 (segment (start 136.5225 93.0275) (end 137.83 91.72) (width 0.2) (layer "F.Cu") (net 22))
 (segment (start 103.8 99) (end 97.936 93.136) (width 0.2) (layer "F.Cu") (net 24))
 (segment (start 118.75 99) (end 156.04 99) (width 0.2) (layer "F.Cu") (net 24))
 (segment (start 118.75 99) (end 103.8 99) (width 0.2) (layer "F.Cu") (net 24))
 (segment (start 97.936 93.136) (end 97.936 28.144) (width 0.2) (layer "F.Cu") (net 24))
 (segment (start 97.936 28.144) (end 99.4 26.68) (width 0.2) (layer "F.Cu") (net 24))
 (segment (start 156.04 99) (end 156.42 99.38) (width 0.2) (layer "F.Cu") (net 24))
 (segment (start 155.7025 54.9275) (end 156.5 54.13) (width 0.2) (layer "F.Cu") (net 4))
 (segment (start 143.66875 54.9275) (end 155.7025 54.9275) (width 0.2) (layer "F.Cu") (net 4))
 (segment (start 143.66875 73.9775) (end 154.9025 73.9775) (width 0.2) (layer "F.Cu") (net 18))
 (segment (start 154.9025 73.9775) (end 156.5 72.38) (width 0.2) (layer "F.Cu") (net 18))
 (segment (start 155.1525 93.0275) (end 156.42 91.76) (width 0.2) (layer "F.Cu") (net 17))
 (segment (start 143.66875 93.0275) (end 155.1525 93.0275) (width 0.2) (layer "F.Cu") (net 17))
 (segment (start 136.57 44.91) (end 118.34 26.68) (width 0.2) (layer "B.Cu") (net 11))
 (segment (start 118.34 26.68) (end 115.475 26.68) (width 0.2) (layer "B.Cu") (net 11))
 (segment (start 136.57 42.37) (end 123.42 29.22) (width 0.2) (layer "F.Cu") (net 10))
 (segment (start 123.42 29.22) (end 114.64 29.22) (width 0.2) (layer "F.Cu") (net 10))
 (segment (start 111.91875 52.3875) (end 111.91875 90.4875) (width 0.2) (layer "B.Cu") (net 6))
 (segment (start 111.91875 52.3875) (end 111.91875 20.07625) (width 0.2) (layer "B.Cu") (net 6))
 (segment (start 111.91875 20.07625) (end 115.475 16.52) (width 0.2) (layer "B.Cu") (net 6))
 (segment (start 130.96875 90.4875) (end 130.96875 52.3875) (width 0.2) (layer "B.Cu") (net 1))
 (segment (start 113.176 20.524) (end 114.64 19.06) (width 0.2) (layer "B.Cu") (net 1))
 (segment (start 113.176 34.59475) (end 113.176 20.524) (width 0.2) (layer "B.Cu") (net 1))
 (segment (start 130.96875 52.3875) (end 113.176 34.59475) (width 0.2) (layer "B.Cu") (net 1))
 (segment (start 113.577 32.20031) (end 113.577 23.498) (width 0.2) (layer "B.Cu") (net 3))
 (segment (start 150.01875 71.4375) (end 150.01875 52.3875) (width 0.2) (layer "B.Cu") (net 3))
 (segment (start 133.76419 52.3875) (end 113.577 32.20031) (width 0.2) (layer "B.Cu") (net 3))
 (segment (start 150.01875 90.4875) (end 150.01875 71.4375) (width 0.2) (layer "B.Cu") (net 3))
 (segment (start 150.01875 52.3875) (end 133.76419 52.3875) (width 0.2) (layer "B.Cu") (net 3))
 (segment (start 113.577 23.498) (end 115.475 21.6) (width 0.2) (layer "B.Cu") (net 3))
 (segment (start 113.577 30.697) (end 114.64 31.76) (width 0.2) (layer "F.Cu") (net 13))
 (segment (start 130.4371 35.67) (end 122.9241 28.157) (width 0.2) (layer "F.Cu") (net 13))
 (segment (start 122.9241 28.157) (end 114.19969 28.157) (width 0.2) (layer "F.Cu") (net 13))
 (segment (start 114.19969 28.157) (end 113.577 28.77969) (width 0.2) (layer "F.Cu") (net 13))
 (segment (start 113.577 28.77969) (end 113.577 30.697) (width 0.2) (layer "F.Cu") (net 13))
 (segment (start 141.05 35.67) (end 130.4371 35.67) (width 0.2) (layer "F.Cu") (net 13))
 (segment (start 132.979 23.077) (end 100.463 23.077) (width 0.2) (layer "F.Cu") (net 14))
 (segment (start 100.463 23.077) (end 99.4 24.14) (width 0.2) (layer "F.Cu") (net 14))
 (segment (start 141.05 40.67) (end 142.351 39.369) (width 0.2) (layer "F.Cu") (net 14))
 (segment (start 142.351 32.449) (end 132.979 23.077) (width 0.2) (layer "F.Cu") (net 14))
 (segment (start 142.351 39.369) (end 142.351 32.449) (width 0.2) (layer "F.Cu") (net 14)))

